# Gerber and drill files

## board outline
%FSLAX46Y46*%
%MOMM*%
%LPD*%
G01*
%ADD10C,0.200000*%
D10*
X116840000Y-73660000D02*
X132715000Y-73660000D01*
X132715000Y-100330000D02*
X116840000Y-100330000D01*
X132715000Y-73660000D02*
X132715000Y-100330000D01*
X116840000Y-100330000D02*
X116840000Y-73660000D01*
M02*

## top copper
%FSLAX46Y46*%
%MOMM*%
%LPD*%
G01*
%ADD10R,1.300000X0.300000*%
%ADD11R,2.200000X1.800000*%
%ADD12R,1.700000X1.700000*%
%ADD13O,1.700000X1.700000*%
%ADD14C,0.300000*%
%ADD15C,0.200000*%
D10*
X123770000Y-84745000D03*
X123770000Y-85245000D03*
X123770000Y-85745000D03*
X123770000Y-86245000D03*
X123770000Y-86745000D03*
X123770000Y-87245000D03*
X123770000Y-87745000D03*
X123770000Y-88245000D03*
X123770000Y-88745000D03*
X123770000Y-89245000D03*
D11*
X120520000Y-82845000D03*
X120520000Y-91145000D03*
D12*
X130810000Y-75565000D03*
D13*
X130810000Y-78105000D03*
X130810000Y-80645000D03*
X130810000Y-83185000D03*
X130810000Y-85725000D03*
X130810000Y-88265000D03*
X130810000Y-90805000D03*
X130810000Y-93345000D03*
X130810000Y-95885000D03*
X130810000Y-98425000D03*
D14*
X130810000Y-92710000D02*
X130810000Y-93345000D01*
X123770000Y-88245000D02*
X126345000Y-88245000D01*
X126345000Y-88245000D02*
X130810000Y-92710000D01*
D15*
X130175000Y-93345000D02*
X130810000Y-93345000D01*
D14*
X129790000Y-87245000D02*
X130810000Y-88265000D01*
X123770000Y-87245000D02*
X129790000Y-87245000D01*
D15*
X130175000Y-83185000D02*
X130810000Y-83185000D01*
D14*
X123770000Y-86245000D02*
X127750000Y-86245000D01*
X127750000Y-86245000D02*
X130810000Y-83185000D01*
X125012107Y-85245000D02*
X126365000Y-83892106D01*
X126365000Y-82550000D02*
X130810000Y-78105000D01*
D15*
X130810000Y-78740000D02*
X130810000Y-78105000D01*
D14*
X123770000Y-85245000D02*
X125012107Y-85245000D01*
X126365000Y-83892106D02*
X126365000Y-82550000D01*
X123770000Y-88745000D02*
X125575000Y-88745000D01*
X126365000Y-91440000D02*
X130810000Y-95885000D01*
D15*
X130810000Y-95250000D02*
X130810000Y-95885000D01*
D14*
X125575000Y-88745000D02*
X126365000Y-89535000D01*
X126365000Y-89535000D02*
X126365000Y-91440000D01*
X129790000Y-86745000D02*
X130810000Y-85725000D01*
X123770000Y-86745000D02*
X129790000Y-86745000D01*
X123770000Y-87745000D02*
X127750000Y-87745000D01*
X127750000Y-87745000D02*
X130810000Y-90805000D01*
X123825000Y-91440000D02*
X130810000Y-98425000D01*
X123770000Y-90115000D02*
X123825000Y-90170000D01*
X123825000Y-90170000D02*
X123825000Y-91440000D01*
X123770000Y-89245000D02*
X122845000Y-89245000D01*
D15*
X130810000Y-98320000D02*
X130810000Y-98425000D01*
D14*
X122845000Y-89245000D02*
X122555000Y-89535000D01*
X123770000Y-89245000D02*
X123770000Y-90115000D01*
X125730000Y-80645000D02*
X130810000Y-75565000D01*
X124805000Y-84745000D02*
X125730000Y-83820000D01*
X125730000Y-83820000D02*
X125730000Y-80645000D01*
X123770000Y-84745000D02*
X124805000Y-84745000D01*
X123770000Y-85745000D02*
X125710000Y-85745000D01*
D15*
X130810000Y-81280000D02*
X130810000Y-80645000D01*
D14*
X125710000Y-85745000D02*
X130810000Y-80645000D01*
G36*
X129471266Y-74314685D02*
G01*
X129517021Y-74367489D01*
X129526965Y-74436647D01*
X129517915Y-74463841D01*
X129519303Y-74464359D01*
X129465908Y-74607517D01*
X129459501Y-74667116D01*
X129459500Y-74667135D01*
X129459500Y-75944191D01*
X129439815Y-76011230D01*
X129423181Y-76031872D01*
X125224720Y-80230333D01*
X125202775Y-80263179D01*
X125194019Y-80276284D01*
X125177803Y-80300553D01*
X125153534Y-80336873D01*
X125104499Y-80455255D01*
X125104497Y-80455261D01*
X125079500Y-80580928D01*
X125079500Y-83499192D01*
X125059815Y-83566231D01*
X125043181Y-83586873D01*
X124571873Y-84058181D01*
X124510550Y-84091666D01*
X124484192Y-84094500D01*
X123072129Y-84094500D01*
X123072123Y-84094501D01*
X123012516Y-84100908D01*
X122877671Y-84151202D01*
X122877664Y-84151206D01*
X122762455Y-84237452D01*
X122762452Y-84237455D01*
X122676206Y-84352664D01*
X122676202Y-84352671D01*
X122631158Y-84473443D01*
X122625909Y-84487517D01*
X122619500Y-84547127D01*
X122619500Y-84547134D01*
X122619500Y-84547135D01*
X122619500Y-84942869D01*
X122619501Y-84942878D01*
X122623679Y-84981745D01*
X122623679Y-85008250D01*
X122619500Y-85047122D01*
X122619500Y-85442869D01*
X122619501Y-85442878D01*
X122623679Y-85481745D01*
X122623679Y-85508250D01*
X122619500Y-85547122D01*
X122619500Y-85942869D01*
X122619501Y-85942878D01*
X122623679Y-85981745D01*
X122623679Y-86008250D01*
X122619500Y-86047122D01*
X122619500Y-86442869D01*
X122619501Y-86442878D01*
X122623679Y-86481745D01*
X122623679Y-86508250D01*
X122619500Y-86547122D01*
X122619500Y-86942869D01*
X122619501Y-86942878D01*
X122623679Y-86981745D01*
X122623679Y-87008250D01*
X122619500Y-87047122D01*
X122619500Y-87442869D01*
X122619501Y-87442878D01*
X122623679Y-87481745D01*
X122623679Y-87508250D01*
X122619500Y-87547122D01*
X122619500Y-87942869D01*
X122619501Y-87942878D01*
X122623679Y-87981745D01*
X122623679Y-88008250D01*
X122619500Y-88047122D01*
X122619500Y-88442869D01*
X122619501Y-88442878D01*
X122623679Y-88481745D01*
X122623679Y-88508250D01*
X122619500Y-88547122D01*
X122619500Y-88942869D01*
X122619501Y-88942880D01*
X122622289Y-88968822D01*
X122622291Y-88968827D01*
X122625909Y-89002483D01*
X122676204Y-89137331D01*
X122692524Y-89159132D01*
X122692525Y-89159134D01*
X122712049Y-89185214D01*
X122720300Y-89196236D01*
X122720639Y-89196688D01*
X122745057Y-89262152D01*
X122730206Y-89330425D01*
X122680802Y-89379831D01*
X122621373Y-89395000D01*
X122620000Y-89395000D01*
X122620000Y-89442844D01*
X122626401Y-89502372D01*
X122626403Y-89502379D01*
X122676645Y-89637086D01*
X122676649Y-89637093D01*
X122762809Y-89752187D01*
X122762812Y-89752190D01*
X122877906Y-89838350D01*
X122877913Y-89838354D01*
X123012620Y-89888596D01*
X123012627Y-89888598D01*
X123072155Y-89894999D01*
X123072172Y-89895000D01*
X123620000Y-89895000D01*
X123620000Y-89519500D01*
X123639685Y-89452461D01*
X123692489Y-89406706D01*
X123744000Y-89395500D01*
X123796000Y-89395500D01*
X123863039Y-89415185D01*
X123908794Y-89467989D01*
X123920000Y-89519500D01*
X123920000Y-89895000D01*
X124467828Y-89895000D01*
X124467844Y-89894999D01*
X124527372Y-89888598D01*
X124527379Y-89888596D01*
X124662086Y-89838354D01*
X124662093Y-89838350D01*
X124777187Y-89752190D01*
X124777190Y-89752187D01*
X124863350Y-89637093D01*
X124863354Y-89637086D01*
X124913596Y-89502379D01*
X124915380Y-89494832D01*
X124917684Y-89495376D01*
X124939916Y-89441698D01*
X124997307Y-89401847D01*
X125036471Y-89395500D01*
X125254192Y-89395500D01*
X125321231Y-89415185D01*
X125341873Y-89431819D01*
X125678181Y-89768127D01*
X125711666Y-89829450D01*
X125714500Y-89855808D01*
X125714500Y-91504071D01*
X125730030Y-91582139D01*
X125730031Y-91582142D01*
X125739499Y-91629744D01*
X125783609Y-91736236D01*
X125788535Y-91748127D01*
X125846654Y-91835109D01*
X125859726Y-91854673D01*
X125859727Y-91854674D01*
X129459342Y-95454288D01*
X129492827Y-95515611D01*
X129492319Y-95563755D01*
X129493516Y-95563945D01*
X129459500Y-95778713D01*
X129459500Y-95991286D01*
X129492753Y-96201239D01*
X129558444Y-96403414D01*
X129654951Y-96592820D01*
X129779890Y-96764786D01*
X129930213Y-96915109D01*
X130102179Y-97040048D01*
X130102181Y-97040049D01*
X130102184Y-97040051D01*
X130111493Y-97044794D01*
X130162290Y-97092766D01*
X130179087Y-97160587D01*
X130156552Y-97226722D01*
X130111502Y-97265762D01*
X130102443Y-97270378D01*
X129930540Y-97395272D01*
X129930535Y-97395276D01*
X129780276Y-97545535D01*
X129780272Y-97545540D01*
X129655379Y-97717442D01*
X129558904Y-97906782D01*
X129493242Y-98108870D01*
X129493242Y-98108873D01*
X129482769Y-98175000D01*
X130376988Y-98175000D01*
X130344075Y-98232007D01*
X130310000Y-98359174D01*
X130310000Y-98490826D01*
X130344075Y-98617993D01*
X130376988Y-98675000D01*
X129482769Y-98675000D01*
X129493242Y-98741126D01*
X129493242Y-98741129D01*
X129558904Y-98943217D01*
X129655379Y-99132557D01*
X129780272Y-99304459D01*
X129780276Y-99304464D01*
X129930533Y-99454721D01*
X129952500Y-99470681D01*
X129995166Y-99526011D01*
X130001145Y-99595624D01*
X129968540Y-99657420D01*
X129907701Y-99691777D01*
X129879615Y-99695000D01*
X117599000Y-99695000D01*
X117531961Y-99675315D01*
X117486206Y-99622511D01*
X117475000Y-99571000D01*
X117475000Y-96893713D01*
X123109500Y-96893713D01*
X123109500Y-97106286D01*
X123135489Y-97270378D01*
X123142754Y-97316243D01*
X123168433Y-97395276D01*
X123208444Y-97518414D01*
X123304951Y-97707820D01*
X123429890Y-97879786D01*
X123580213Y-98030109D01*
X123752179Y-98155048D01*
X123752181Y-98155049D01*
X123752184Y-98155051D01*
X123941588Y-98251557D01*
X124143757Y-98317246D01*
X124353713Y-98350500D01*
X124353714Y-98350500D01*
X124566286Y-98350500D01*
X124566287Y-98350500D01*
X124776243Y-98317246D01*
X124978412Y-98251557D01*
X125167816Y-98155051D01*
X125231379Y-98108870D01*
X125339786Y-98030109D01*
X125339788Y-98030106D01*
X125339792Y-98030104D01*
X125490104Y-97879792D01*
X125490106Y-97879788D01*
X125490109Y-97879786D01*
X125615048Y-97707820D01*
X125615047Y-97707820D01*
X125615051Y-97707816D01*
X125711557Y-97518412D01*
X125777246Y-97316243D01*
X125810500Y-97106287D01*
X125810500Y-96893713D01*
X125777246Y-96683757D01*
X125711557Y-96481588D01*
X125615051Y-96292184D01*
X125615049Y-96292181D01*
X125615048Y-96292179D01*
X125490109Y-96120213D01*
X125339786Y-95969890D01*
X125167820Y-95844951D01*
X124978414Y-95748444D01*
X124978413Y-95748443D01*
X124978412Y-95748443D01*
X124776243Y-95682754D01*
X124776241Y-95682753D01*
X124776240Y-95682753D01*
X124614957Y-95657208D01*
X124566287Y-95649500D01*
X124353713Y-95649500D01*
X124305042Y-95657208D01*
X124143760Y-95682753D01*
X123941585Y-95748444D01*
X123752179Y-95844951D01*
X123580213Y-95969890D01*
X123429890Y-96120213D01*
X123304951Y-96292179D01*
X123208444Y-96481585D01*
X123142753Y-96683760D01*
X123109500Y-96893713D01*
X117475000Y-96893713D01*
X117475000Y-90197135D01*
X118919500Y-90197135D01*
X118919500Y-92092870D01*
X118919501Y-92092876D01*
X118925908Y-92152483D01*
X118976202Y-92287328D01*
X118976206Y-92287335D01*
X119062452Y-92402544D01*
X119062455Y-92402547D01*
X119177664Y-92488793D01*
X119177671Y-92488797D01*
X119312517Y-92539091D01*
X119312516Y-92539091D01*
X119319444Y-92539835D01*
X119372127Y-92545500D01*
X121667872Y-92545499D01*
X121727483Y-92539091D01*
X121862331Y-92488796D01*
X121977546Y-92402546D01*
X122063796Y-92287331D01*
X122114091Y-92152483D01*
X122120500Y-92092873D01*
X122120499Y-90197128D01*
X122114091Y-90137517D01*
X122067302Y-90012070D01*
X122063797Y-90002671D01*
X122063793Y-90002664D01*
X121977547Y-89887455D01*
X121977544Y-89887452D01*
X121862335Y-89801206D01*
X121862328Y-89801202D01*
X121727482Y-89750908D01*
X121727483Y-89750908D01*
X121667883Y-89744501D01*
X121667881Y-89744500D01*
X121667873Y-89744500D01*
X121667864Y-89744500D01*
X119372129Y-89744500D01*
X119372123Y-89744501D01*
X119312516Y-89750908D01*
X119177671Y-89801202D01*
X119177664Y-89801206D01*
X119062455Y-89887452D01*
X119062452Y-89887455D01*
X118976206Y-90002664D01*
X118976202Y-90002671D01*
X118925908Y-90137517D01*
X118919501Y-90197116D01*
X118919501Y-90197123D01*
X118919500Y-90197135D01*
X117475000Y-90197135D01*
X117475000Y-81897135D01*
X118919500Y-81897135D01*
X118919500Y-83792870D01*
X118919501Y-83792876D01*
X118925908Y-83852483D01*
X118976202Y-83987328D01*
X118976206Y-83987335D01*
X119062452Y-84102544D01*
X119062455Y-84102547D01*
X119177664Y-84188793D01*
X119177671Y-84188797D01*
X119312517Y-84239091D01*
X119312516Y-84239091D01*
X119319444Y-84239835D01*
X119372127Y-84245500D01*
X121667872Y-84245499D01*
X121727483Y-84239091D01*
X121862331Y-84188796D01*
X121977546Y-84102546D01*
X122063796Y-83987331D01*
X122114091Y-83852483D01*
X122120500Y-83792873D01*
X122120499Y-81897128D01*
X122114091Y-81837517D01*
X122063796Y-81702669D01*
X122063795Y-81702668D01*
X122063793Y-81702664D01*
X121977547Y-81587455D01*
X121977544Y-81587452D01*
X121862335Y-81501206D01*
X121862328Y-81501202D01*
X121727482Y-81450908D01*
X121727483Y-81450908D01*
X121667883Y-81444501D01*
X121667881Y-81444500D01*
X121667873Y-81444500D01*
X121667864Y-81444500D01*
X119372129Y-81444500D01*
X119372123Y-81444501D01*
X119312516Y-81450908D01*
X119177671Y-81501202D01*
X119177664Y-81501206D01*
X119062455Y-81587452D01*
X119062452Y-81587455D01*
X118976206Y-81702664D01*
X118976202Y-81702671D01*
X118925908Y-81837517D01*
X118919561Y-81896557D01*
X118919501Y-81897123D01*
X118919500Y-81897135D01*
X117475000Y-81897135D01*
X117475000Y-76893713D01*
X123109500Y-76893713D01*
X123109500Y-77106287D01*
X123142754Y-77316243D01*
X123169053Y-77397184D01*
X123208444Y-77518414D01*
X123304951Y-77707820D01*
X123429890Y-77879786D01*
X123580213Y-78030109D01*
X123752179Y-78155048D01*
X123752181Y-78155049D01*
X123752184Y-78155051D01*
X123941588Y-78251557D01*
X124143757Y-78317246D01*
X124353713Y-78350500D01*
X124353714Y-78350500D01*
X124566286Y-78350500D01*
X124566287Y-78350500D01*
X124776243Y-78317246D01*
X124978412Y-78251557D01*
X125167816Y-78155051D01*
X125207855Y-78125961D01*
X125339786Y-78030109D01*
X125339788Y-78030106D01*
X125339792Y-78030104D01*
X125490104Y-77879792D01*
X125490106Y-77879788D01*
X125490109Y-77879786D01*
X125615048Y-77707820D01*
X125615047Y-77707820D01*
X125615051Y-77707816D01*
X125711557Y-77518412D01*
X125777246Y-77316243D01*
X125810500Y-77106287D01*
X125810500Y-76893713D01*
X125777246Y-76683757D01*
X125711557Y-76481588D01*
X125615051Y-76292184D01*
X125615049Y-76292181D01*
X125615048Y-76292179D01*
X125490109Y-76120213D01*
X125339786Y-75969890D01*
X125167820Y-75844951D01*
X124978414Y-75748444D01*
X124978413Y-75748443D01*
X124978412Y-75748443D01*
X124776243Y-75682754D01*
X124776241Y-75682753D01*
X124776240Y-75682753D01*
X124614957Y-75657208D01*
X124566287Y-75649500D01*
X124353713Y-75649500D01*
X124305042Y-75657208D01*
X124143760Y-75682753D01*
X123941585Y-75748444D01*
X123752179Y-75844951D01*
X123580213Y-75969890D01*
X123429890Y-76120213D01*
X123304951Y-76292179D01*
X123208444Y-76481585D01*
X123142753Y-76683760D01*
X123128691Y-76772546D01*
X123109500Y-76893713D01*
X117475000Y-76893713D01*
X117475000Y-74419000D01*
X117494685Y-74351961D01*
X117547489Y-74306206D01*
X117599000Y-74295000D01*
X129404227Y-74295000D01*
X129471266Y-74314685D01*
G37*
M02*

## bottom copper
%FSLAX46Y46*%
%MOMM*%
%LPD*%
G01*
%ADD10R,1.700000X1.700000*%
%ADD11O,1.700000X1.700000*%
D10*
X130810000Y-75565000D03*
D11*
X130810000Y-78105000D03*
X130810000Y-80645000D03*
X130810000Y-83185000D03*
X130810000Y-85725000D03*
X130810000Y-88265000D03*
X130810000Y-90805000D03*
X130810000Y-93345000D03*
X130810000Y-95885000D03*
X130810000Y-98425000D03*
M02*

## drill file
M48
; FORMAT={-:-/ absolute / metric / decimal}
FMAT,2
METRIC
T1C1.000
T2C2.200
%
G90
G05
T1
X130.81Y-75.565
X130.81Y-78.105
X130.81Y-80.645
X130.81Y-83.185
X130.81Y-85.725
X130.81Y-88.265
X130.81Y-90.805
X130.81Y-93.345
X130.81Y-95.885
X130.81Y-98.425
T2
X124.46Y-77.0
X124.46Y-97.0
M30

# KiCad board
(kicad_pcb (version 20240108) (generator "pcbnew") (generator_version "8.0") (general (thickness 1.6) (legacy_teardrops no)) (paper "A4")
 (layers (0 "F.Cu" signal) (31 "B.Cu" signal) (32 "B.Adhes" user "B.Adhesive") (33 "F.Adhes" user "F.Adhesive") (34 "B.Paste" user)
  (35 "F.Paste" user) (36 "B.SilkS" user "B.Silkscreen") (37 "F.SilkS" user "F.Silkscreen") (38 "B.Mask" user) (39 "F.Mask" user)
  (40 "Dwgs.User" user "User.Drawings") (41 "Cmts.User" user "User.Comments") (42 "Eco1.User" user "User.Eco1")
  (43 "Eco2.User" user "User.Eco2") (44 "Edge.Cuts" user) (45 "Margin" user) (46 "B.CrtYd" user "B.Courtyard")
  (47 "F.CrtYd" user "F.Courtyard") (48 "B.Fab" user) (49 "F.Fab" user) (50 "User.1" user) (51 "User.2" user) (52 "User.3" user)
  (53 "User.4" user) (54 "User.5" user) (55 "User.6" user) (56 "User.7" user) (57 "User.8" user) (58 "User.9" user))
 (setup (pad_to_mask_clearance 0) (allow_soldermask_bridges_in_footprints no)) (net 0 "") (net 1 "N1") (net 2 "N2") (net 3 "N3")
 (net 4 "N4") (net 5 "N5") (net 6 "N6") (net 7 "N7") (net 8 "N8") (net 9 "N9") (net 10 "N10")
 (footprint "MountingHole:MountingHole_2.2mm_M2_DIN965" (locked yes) (layer "F.Cu") (at 124.46 97)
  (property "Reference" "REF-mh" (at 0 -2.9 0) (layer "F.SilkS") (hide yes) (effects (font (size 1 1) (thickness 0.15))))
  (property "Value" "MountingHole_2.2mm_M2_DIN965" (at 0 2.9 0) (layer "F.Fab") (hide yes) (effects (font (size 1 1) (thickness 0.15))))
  (pad "" np_thru_hole circle (at 0 0) (size 2.2 2.2) (drill 2.2) (layers "F&B.Cu" "*.Mask")))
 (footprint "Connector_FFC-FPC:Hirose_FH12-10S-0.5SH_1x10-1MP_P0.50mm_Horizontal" (layer "F.Cu") (at 121.92 86.995 -90)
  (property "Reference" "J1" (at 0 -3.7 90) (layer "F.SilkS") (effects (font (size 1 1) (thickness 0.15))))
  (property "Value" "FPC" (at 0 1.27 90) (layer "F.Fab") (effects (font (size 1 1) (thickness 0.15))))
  (pad "1" smd rect (at -2.25 -1.85 270) (size 0.3 1.3) (layers "F.Cu" "F.Paste" "F.Mask") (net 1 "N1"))
  (pad "2" smd rect (at -1.75 -1.85 270) (size 0.3 1.3) (layers "F.Cu" "F.Paste" "F.Mask") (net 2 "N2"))
  (pad "3" smd rect (at -1.25 -1.85 270) (size 0.3 1.3) (layers "F.Cu" "F.Paste" "F.Mask") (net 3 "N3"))
  (pad "4" smd rect (at -0.75 -1.85 270) (size 0.3 1.3) (layers "F.Cu" "F.Paste" "F.Mask") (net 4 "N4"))
  (pad "5" smd rect (at -0.25 -1.85 270) (size 0.3 1.3) (layers "F.Cu" "F.Paste" "F.Mask") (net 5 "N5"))
  (pad "6" smd rect (at 0.25 -1.85 270) (size 0.3 1.3) (layers "F.Cu" "F.Paste" "F.Mask") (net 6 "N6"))
  (pad "7" smd rect (at 0.75 -1.85 270) (size 0.3 1.3) (layers "F.Cu" "F.Paste" "F.Mask") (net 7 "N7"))
  (pad "8" smd rect (at 1.25 -1.85 270) (size 0.3 1.3) (layers "F.Cu" "F.Paste" "F.Mask") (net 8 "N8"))
  (pad "9" smd rect (at 1.75 -1.85 270) (size 0.3 1.3) (layers "F.Cu" "F.Paste" "F.Mask") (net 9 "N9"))
  (pad "10" smd rect (at 2.25 -1.85 270) (size 0.3 1.3) (layers "F.Cu" "F.Paste" "F.Mask") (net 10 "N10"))
  (pad "MP" smd rect (at -4.15 1.4 270) (size 1.8 2.2) (layers "F.Cu" "F.Paste" "F.Mask"))
  (pad "MP" smd rect (at 4.15 1.4 270) (size 1.8 2.2) (layers "F.Cu" "F.Paste" "F.Mask")))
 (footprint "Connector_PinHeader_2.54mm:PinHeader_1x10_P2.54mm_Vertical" (layer "F.Cu") (at 130.81 75.565)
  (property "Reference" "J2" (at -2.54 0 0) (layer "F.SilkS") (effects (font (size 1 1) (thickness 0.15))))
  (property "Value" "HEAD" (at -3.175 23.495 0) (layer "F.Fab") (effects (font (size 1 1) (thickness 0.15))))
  (pad "1" thru_hole rect (at 0 0) (size 1.7 1.7) (drill 1) (layers "*.Cu" "*.Mask") (remove_unused_layers no) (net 1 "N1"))
  (pad "2" thru_hole oval (at 0 2.54) (size 1.7 1.7) (drill 1) (layers "*.Cu" "*.Mask") (remove_unused_layers no) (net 2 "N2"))
  (pad "3" thru_hole oval (at 0 5.08) (size 1.7 1.7) (drill 1) (layers "*.Cu" "*.Mask") (remove_unused_layers no) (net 3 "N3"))
  (pad "4" thru_hole oval (at 0 7.62) (size 1.7 1.7) (drill 1) (layers "*.Cu" "*.Mask") (remove_unused_layers no) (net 4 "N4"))
  (pad "5" thru_hole oval (at 0 10.16) (size 1.7 1.7) (drill 1) (layers "*.Cu" "*.Mask") (remove_unused_layers no) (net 5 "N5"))
  (pad "6" thru_hole oval (at 0 12.7) (size 1.7 1.7) (drill 1) (layers "*.Cu" "*.Mask") (remove_unused_layers no) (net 6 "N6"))
  (pad "7" thru_hole oval (at 0 15.24) (size 1.7 1.7) (drill 1) (layers "*.Cu" "*.Mask") (remove_unused_layers no) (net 7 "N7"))
  (pad "8" thru_hole oval (at 0 17.78) (size 1.7 1.7) (drill 1) (layers "*.Cu" "*.Mask") (remove_unused_layers no) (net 8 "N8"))
  (pad "9" thru_hole oval (at 0 20.32) (size 1.7 1.7) (drill 1) (layers "*.Cu" "*.Mask") (remove_unused_layers no) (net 9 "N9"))
  (pad "10" thru_hole oval (at 0 22.86) (size 1.7 1.7) (drill 1) (layers "*.Cu" "*.Mask") (remove_unused_layers no) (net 10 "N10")))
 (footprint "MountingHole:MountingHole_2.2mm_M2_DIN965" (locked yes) (layer "F.Cu") (at 124.46 77)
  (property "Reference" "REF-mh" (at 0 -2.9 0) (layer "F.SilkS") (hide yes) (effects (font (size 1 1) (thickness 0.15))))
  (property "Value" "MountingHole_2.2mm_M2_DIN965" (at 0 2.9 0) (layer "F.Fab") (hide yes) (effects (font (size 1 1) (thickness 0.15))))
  (pad "" np_thru_hole circle (at 0 0) (size 2.2 2.2) (drill 2.2) (layers "*.Cu" "*.Mask")))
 (gr_line (start 116.84 73.66) (end 132.715 73.66) (locked yes) (stroke (width 0.2) (type default)) (layer "Edge.Cuts"))
 (gr_line (start 132.715 100.33) (end 116.84 100.33) (locked yes) (stroke (width 0.2) (type default)) (layer "Edge.Cuts"))
 (gr_line (start 132.715 73.66) (end 132.715 100.33) (locked yes) (stroke (width 0.2) (type default)) (layer "Edge.Cuts"))
 (gr_line (start 116.84 100.33) (end 116.84 73.66) (locked yes) (stroke (width 0.2) (type default)) (layer "Edge.Cuts"))
 (segment (start 130.81 92.71) (end 130.81 93.345) (width 0.3) (layer "F.Cu") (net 8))
 (segment (start 123.77 88.245) (end 126.345 88.245) (width 0.3) (layer "F.Cu") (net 8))
 (segment (start 126.345 88.245) (end 130.81 92.71) (width 0.3) (layer "F.Cu") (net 8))
 (segment (start 130.175 93.345) (end 130.81 93.345) (width 0.2) (layer "F.Cu") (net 8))
 (segment (start 129.79 87.245) (end 130.81 88.265) (width 0.3) (layer "F.Cu") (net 6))
 (segment (start 123.77 87.245) (end 129.79 87.245) (width 0.3) (layer "F.Cu") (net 6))
 (segment (start 130.175 83.185) (end 130.81 83.185) (width 0.2) (layer "F.Cu") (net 4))
 (segment (start 123.77 86.245) (end 127.75 86.245) (width 0.3) (layer "F.Cu") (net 4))
 (segment (start 127.75 86.245) (end 130.81 83.185) (width 0.3) (layer "F.Cu") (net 4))
 (segment (start 125.012107 85.245) (end 126.365 83.892106) (width 0.3) (layer "F.Cu") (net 2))
 (segment (start 126.365 82.55) (end 130.81 78.105) (width 0.3) (layer "F.Cu") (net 2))
 (segment (start 130.81 78.74) (end 130.81 78.105) (width 0.2) (layer "F.Cu") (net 2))
 (segment (start 123.77 85.245) (end 125.012107 85.245) (width 0.3) (layer "F.Cu") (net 2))
 (segment (start 126.365 83.892106) (end 126.365 82.55) (width 0.3) (layer "F.Cu") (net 2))
 (segment (start 123.77 88.745) (end 125.575 88.745) (width 0.3) (layer "F.Cu") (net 9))
 (segment (start 126.365 91.44) (end 130.81 95.885) (width 0.3) (layer "F.Cu") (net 9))
 (segment (start 130.81 95.25) (end 130.81 95.885) (width 0.2) (layer "F.Cu") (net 9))
 (segment (start 125.575 88.745) (end 126.365 89.535) (width 0.3) (layer "F.Cu") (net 9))
 (segment (start 126.365 89.535) (end 126.365 91.44) (width 0.3) (layer "F.Cu") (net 9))
 (segment (start 129.79 86.745) (end 130.81 85.725) (width 0.3) (layer "F.Cu") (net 5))
 (segment (start 123.77 86.745) (end 129.79 86.745) (width 0.3) (layer "F.Cu") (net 5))
 (segment (start 123.77 87.745) (end 127.75 87.745) (width 0.3) (layer "F.Cu") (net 7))
 (segment (start 127.75 87.745) (end 130.81 90.805) (width 0.3) (layer "F.Cu") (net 7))
 (segment (start 123.825 91.44) (end 130.81 98.425) (width 0.3) (layer "F.Cu") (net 10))
 (segment (start 123.77 90.115) (end 123.825 90.17) (width 0.3) (layer "F.Cu") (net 10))
 (segment (start 123.825 90.17) (end 123.825 91.44) (width 0.3) (layer "F.Cu") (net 10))
 (segment (start 123.77 89.245) (end 122.845 89.245) (width 0.3) (layer "F.Cu") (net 10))
 (segment (start 130.81 98.32) (end 130.81 98.425) (width 0.2) (layer "F.Cu") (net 10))
 (segment (start 122.845 89.245) (end 122.555 89.535) (width 0.3) (layer "F.Cu") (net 10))
 (segment (start 123.77 89.245) (end 123.77 90.115) (width 0.3) (layer "F.Cu") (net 10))
 (segment (start 125.73 80.645) (end 130.81 75.565) (width 0.3) (layer "F.Cu") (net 1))
 (segment (start 124.805 84.745) (end 125.73 83.82) (width 0.3) (layer "F.Cu") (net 1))
 (segment (start 125.73 83.82) (end 125.73 80.645) (width 0.3) (layer "F.Cu") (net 1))
 (segment (start 123.77 84.745) (end 124.805 84.745) (width 0.3) (layer "F.Cu") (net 1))
 (segment (start 123.77 85.745) (end 125.71 85.745) (width 0.3) (layer "F.Cu") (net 3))
 (segment (start 130.81 81.28) (end 130.81 80.645) (width 0.2) (layer "F.Cu") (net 3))
 (segment (start 125.71 85.745) (end 130.81 80.645) (width 0.3) (layer "F.Cu") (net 3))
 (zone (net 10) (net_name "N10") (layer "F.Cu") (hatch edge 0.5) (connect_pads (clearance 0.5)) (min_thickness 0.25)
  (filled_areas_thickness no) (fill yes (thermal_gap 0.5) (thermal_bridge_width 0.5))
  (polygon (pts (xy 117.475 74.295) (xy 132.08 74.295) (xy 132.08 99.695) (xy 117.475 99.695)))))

